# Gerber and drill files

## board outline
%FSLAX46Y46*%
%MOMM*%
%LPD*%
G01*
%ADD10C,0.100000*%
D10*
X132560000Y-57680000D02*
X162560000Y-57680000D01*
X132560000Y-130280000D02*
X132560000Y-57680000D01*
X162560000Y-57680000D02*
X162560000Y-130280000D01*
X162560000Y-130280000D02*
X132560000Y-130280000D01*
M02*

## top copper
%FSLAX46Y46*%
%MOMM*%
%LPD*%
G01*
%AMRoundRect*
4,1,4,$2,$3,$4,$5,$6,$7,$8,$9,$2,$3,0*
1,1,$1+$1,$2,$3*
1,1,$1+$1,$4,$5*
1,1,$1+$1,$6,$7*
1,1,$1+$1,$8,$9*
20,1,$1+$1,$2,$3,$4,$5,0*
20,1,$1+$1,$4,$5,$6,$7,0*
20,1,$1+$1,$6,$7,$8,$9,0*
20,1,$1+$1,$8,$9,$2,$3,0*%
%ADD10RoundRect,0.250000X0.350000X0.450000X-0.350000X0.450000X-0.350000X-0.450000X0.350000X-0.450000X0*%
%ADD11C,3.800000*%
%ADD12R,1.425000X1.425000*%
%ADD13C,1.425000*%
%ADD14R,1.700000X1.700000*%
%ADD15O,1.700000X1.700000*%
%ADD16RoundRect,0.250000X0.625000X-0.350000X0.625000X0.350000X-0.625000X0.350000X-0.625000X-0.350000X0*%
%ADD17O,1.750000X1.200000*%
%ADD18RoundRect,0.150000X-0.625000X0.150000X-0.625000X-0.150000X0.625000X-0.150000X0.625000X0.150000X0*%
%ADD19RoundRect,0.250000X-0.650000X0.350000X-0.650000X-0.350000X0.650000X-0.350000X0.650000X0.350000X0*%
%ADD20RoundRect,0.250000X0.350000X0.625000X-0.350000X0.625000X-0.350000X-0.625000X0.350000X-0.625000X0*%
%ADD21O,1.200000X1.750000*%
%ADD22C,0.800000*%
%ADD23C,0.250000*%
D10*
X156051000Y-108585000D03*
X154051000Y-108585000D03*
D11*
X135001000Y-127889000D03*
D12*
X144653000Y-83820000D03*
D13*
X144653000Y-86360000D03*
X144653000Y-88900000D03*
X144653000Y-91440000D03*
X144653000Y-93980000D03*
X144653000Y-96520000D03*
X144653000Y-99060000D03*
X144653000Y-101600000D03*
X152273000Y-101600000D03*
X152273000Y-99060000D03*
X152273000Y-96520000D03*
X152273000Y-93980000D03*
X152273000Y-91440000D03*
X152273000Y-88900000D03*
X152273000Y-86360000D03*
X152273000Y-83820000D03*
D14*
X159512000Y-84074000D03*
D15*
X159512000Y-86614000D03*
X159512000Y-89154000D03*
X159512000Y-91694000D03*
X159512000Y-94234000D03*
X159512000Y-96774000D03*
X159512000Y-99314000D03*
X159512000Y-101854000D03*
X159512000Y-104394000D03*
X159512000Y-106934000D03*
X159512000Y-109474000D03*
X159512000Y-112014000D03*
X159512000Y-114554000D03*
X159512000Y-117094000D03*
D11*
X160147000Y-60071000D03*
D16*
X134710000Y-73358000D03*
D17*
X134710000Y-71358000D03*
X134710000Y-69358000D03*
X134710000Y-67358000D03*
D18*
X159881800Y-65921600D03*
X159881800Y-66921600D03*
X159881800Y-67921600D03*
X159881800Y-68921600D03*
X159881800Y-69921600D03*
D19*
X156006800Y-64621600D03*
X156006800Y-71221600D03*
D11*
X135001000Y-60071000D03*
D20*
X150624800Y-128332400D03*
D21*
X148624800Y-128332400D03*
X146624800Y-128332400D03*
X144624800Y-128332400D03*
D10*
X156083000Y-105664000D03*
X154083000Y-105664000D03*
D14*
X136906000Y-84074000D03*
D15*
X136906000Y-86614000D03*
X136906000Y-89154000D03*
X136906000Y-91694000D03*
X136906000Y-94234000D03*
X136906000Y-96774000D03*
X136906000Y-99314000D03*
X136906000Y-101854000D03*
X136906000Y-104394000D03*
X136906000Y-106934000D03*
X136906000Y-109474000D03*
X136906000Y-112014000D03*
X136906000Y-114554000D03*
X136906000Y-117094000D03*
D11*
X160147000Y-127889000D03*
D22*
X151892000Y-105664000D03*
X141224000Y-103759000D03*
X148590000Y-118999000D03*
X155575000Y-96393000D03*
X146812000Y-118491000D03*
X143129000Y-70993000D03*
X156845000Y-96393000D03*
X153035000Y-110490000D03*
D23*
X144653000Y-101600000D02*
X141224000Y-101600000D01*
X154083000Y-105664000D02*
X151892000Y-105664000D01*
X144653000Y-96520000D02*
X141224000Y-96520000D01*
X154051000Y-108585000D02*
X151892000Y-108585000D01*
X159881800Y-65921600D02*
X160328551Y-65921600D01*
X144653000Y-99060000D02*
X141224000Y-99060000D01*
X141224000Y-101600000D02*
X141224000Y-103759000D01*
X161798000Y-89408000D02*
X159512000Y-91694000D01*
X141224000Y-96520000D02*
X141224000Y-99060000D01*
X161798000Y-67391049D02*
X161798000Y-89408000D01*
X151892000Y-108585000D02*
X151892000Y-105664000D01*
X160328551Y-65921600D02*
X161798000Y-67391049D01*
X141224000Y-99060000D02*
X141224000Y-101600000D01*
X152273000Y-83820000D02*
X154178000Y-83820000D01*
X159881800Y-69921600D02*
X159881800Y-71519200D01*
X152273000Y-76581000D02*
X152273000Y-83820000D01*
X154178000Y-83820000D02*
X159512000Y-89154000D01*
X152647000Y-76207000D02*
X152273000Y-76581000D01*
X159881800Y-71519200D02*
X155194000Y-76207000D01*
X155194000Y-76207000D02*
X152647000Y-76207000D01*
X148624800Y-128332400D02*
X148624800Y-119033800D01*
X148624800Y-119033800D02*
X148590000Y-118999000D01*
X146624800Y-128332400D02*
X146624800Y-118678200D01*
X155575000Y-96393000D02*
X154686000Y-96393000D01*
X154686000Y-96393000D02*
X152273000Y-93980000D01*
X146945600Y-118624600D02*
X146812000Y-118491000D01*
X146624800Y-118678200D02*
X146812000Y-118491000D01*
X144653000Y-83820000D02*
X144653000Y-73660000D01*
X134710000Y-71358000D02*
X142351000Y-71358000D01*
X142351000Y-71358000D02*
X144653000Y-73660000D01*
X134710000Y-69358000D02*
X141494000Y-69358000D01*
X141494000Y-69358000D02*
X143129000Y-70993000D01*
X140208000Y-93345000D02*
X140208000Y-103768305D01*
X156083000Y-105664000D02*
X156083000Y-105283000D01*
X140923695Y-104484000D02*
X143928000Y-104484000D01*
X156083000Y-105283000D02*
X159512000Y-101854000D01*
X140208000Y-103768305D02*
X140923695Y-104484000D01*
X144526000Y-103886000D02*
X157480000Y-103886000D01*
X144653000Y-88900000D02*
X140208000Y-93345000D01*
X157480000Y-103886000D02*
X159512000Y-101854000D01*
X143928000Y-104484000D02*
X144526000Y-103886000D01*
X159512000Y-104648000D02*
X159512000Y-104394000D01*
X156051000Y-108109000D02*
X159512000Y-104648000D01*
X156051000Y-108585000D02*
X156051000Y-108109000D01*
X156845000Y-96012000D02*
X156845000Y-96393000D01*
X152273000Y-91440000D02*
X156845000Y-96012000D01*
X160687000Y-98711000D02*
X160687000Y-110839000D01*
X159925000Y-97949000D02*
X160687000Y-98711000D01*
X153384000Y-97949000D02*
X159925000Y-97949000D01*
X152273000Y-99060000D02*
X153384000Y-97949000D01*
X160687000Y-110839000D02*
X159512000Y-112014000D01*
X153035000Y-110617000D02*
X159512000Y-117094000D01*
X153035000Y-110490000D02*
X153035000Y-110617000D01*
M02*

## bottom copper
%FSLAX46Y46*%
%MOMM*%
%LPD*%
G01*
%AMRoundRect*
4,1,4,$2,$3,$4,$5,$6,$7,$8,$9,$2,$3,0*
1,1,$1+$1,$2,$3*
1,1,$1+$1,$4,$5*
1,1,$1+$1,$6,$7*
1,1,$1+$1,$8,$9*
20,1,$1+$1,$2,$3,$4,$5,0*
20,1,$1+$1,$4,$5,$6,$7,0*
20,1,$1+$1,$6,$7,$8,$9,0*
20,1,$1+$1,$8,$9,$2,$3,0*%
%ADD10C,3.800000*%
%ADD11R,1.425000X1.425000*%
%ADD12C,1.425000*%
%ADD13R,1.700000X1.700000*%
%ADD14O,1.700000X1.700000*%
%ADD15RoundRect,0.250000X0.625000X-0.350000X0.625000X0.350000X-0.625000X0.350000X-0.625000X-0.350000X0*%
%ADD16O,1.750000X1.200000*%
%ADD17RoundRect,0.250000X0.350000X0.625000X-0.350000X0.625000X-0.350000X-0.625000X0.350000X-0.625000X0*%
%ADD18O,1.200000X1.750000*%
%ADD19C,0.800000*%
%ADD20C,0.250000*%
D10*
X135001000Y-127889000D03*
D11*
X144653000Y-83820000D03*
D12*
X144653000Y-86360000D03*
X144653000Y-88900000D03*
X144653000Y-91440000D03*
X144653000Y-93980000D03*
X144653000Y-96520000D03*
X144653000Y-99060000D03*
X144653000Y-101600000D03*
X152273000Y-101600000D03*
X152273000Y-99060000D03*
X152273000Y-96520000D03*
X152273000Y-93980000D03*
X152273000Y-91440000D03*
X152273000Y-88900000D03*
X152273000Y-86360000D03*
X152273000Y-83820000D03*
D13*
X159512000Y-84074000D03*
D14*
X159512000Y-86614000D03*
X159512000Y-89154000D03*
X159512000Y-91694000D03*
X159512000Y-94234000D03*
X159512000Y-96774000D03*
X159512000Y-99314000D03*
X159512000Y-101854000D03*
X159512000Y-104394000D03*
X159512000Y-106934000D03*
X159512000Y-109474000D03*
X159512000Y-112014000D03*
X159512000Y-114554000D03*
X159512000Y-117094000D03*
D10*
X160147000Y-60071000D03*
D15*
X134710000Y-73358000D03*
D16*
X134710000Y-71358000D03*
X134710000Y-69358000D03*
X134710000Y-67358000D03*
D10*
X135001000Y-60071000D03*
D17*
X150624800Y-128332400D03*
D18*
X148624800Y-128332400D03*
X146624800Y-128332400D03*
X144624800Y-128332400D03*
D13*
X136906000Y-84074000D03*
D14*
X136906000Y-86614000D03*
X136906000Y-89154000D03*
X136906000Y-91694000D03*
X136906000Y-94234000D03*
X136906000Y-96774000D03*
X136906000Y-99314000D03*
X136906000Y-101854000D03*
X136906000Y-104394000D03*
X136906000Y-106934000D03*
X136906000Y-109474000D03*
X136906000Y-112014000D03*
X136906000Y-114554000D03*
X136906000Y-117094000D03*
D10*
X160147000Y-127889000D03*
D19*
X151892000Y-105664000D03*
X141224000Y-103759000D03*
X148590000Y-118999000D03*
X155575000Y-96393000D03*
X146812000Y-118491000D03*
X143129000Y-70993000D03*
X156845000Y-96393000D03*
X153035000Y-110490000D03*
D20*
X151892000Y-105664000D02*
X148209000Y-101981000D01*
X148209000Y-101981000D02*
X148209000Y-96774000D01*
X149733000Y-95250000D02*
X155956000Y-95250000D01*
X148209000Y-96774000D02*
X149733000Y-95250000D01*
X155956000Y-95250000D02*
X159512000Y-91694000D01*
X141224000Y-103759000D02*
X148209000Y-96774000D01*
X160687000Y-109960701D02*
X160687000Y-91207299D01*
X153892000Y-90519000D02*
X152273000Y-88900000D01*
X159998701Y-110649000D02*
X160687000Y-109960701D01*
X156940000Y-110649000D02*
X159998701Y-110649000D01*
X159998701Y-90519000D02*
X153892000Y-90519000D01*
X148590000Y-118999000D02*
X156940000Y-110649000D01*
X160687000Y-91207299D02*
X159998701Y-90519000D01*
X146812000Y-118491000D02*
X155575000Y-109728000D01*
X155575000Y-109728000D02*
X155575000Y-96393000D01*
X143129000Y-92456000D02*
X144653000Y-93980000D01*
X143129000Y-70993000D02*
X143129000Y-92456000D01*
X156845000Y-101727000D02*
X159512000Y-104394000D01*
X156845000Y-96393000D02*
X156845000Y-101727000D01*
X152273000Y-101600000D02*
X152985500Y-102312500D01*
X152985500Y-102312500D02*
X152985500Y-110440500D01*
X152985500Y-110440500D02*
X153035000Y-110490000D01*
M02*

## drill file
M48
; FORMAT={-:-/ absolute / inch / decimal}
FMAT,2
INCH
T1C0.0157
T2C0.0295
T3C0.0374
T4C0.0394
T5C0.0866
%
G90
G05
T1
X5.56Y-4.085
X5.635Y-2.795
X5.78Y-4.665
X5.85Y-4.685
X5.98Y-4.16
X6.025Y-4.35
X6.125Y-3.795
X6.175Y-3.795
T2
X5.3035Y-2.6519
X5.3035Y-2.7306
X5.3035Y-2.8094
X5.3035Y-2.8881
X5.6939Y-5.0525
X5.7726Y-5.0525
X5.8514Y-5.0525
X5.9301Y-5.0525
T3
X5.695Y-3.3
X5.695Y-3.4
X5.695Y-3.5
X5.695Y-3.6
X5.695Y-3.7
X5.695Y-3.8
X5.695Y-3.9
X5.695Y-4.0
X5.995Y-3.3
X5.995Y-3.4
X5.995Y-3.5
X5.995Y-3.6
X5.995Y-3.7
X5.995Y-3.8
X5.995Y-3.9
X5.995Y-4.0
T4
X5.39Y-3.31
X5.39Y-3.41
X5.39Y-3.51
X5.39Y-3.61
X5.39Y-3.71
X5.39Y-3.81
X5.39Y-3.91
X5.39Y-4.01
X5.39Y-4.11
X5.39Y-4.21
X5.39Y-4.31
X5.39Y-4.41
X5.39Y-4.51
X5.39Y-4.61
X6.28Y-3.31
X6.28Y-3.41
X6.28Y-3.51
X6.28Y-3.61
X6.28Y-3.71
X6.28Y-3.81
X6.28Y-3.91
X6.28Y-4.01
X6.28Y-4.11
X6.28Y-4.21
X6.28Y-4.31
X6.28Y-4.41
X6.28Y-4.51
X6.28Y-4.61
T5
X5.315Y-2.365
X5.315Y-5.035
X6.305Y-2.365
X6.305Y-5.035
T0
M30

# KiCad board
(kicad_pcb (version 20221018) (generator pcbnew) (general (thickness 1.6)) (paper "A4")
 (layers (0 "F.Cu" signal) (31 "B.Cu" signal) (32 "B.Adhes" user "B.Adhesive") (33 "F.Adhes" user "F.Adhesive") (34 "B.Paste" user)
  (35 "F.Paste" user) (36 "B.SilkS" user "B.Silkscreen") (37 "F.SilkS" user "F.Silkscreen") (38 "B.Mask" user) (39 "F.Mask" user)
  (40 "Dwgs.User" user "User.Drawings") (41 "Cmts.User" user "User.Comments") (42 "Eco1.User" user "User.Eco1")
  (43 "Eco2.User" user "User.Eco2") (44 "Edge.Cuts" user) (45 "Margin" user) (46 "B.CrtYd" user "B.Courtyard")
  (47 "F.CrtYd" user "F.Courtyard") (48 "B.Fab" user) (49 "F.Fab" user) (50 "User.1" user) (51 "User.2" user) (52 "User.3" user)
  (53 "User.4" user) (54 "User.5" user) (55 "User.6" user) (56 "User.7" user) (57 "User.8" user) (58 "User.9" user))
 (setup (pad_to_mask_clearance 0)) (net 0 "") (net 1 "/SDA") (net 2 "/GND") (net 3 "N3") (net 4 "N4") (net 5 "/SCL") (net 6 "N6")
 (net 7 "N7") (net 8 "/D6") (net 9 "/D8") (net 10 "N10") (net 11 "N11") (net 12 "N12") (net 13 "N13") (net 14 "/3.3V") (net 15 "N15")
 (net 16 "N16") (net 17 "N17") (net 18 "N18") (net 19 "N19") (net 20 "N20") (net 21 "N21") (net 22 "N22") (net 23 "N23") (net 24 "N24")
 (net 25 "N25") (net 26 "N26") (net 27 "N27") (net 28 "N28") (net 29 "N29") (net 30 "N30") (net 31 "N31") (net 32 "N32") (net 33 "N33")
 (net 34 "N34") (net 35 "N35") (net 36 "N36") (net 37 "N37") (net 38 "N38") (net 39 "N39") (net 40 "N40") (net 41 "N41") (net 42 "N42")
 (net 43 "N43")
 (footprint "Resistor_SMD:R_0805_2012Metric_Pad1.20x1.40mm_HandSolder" (layer "F.Cu") (at 155.051 108.585 180)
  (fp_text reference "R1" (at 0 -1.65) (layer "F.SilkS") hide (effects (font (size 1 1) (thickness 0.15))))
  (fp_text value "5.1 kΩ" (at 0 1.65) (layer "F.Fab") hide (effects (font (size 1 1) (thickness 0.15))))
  (pad "1" smd roundrect (at -1 0 180) (size 1.2 1.4) (layers "F.Cu" "F.Paste" "F.Mask") (roundrect_rratio 0.2083333333) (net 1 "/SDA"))
  (pad "2" smd roundrect (at 1 0 180) (size 1.2 1.4) (layers "F.Cu" "F.Paste" "F.Mask") (roundrect_rratio 0.2083333333) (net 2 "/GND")))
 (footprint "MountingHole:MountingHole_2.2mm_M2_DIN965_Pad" (layer "F.Cu") (at 135.001 127.889)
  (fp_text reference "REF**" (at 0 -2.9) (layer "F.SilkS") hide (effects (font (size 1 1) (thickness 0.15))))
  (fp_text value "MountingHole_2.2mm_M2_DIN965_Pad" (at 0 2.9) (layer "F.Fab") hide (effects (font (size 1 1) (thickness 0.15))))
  (pad "1" thru_hole circle (at 0 0) (size 3.8 3.8) (drill 2.2) (layers "*.Cu" "*.Mask")))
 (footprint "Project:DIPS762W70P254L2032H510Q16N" (layer "F.Cu") (at 144.653 83.82)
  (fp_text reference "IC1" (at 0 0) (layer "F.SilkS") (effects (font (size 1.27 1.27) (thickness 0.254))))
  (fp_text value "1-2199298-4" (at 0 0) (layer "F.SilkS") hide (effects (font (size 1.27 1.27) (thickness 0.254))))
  (pad "1" thru_hole rect (at 0 0) (size 1.425 1.425) (drill 0.95) (layers "*.Cu" "*.Mask") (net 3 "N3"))
  (pad "2" thru_hole circle (at 0 2.54) (size 1.425 1.425) (drill 0.95) (layers "*.Cu" "*.Mask") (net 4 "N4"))
  (pad "3" thru_hole circle (at 0 5.08) (size 1.425 1.425) (drill 0.95) (layers "*.Cu" "*.Mask") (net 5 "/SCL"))
  (pad "4" thru_hole circle (at 0 7.62) (size 1.425 1.425) (drill 0.95) (layers "*.Cu" "*.Mask") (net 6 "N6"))
  (pad "5" thru_hole circle (at 0 10.16) (size 1.425 1.425) (drill 0.95) (layers "*.Cu" "*.Mask") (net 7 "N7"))
  (pad "6" thru_hole circle (at 0 12.7) (size 1.425 1.425) (drill 0.95) (layers "*.Cu" "*.Mask") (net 2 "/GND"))
  (pad "7" thru_hole circle (at 0 15.24) (size 1.425 1.425) (drill 0.95) (layers "*.Cu" "*.Mask") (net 2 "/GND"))
  (pad "8" thru_hole circle (at 0 17.78) (size 1.425 1.425) (drill 0.95) (layers "*.Cu" "*.Mask") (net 2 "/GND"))
  (pad "9" thru_hole circle (at 7.62 17.78) (size 1.425 1.425) (drill 0.95) (layers "*.Cu" "*.Mask") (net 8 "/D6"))
  (pad "10" thru_hole circle (at 7.62 15.24) (size 1.425 1.425) (drill 0.95) (layers "*.Cu" "*.Mask") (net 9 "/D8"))
  (pad "11" thru_hole circle (at 7.62 12.7) (size 1.425 1.425) (drill 0.95) (layers "*.Cu" "*.Mask") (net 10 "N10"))
  (pad "12" thru_hole circle (at 7.62 10.16) (size 1.425 1.425) (drill 0.95) (layers "*.Cu" "*.Mask") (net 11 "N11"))
  (pad "13" thru_hole circle (at 7.62 7.62) (size 1.425 1.425) (drill 0.95) (layers "*.Cu" "*.Mask") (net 1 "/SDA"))
  (pad "14" thru_hole circle (at 7.62 5.08) (size 1.425 1.425) (drill 0.95) (layers "*.Cu" "*.Mask") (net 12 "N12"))
  (pad "15" thru_hole circle (at 7.62 2.54) (size 1.425 1.425) (drill 0.95) (layers "*.Cu" "*.Mask") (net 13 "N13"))
  (pad "16" thru_hole circle (at 7.62 0) (size 1.425 1.425) (drill 0.95) (layers "*.Cu" "*.Mask") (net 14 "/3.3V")))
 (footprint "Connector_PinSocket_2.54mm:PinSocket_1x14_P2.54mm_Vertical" (layer "F.Cu") (at 159.512 84.074)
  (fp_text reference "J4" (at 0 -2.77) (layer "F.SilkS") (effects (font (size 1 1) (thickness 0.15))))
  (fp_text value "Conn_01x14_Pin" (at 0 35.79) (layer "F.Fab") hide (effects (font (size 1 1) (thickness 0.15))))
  (pad "1" thru_hole rect (at 0 0) (size 1.7 1.7) (drill 1) (layers "*.Cu" "*.Mask") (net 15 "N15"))
  (pad "2" thru_hole oval (at 0 2.54) (size 1.7 1.7) (drill 1) (layers "*.Cu" "*.Mask") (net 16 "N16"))
  (pad "3" thru_hole oval (at 0 5.08) (size 1.7 1.7) (drill 1) (layers "*.Cu" "*.Mask") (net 14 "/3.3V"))
  (pad "4" thru_hole oval (at 0 7.62) (size 1.7 1.7) (drill 1) (layers "*.Cu" "*.Mask") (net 2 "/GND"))
  (pad "5" thru_hole oval (at 0 10.16) (size 1.7 1.7) (drill 1) (layers "*.Cu" "*.Mask") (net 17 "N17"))
  (pad "6" thru_hole oval (at 0 12.7) (size 1.7 1.7) (drill 1) (layers "*.Cu" "*.Mask") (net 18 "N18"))
  (pad "7" thru_hole oval (at 0 15.24) (size 1.7 1.7) (drill 1) (layers "*.Cu" "*.Mask") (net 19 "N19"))
  (pad "8" thru_hole oval (at 0 17.78) (size 1.7 1.7) (drill 1) (layers "*.Cu" "*.Mask") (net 5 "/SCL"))
  (pad "9" thru_hole oval (at 0 20.32) (size 1.7 1.7) (drill 1) (layers "*.Cu" "*.Mask") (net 1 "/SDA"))
  (pad "10" thru_hole oval (at 0 22.86) (size 1.7 1.7) (drill 1) (layers "*.Cu" "*.Mask") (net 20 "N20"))
  (pad "11" thru_hole oval (at 0 25.4) (size 1.7 1.7) (drill 1) (layers "*.Cu" "*.Mask") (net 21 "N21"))
  (pad "12" thru_hole oval (at 0 27.94) (size 1.7 1.7) (drill 1) (layers "*.Cu" "*.Mask") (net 9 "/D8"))
  (pad "13" thru_hole oval (at 0 30.48) (size 1.7 1.7) (drill 1) (layers "*.Cu" "*.Mask") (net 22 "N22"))
  (pad "14" thru_hole oval (at 0 33.02) (size 1.7 1.7) (drill 1) (layers "*.Cu" "*.Mask") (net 8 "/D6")))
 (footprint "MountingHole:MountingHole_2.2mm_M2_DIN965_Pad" (layer "F.Cu") (at 160.147 60.071)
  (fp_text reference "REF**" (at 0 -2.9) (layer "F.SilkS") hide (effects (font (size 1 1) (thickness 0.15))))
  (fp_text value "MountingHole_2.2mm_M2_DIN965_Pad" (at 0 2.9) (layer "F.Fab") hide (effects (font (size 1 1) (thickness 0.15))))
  (pad "1" thru_hole circle (at 0 0) (size 3.8 3.8) (drill 2.2) (layers "*.Cu" "*.Mask")))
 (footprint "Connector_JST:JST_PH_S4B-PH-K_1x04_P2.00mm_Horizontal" (layer "F.Cu") (at 134.71 73.358 90)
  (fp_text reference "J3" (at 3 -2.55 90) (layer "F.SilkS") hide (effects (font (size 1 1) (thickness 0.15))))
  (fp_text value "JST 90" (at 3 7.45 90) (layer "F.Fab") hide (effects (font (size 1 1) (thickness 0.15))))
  (pad "1" thru_hole roundrect (at 0 0 90) (size 1.2 1.75) (drill 0.75) (layers "*.Cu" "*.Mask") (roundrect_rratio 0.2083333333)
   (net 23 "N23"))
  (pad "2" thru_hole oval (at 2 0 90) (size 1.2 1.75) (drill 0.75) (layers "*.Cu" "*.Mask") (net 3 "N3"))
  (pad "3" thru_hole oval (at 4 0 90) (size 1.2 1.75) (drill 0.75) (layers "*.Cu" "*.Mask") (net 7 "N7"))
  (pad "4" thru_hole oval (at 6 0 90) (size 1.2 1.75) (drill 0.75) (layers "*.Cu" "*.Mask") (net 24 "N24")))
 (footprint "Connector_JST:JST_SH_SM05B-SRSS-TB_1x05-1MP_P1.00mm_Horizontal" (layer "F.Cu") (at 157.8818 67.9216 -90)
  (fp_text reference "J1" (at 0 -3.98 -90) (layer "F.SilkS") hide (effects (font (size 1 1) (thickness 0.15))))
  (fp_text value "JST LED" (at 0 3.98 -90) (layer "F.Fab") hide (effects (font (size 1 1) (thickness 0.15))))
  (pad "1" smd roundrect (at -2 -2 270) (size 0.6 1.55) (layers "F.Cu" "F.Paste" "F.Mask") (roundrect_rratio 0.25) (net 2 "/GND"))
  (pad "2" smd roundrect (at -1 -2 270) (size 0.6 1.55) (layers "F.Cu" "F.Paste" "F.Mask") (roundrect_rratio 0.25) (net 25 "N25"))
  (pad "3" smd roundrect (at 0 -2 270) (size 0.6 1.55) (layers "F.Cu" "F.Paste" "F.Mask") (roundrect_rratio 0.25) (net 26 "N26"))
  (pad "4" smd roundrect (at 1 -2 270) (size 0.6 1.55) (layers "F.Cu" "F.Paste" "F.Mask") (roundrect_rratio 0.25) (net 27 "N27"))
  (pad "5" smd roundrect (at 2 -2 270) (size 0.6 1.55) (layers "F.Cu" "F.Paste" "F.Mask") (roundrect_rratio 0.25) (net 14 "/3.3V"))
  (pad "MP" smd roundrect (at -3.3 1.875 270) (size 1.2 1.8) (layers "F.Cu" "F.Paste" "F.Mask") (roundrect_rratio 0.2083333333))
  (pad "MP" smd roundrect (at 3.3 1.875 270) (size 1.2 1.8) (layers "F.Cu" "F.Paste" "F.Mask") (roundrect_rratio 0.2083333333)))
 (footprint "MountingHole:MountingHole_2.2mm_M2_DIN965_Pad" (layer "F.Cu") (at 135.001 60.071)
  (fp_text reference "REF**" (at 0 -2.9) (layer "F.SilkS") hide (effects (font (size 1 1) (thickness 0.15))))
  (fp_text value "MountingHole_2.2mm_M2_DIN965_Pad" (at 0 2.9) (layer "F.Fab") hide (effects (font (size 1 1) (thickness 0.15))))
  (pad "1" thru_hole circle (at 0 0) (size 3.8 3.8) (drill 2.2) (layers "*.Cu" "*.Mask")))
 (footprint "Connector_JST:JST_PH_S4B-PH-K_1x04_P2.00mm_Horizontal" (layer "F.Cu") (at 150.6248 128.3324 180)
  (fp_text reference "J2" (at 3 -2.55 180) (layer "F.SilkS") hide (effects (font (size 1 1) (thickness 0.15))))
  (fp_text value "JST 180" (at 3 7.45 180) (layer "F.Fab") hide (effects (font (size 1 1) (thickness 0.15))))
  (pad "1" thru_hole roundrect (at 0 0 180) (size 1.2 1.75) (drill 0.75) (layers "*.Cu" "*.Mask") (roundrect_rratio 0.2083333333)
   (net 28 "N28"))
  (pad "2" thru_hole oval (at 2 0 180) (size 1.2 1.75) (drill 0.75) (layers "*.Cu" "*.Mask") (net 12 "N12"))
  (pad "3" thru_hole oval (at 4 0 180) (size 1.2 1.75) (drill 0.75) (layers "*.Cu" "*.Mask") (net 11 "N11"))
  (pad "4" thru_hole oval (at 6 0 180) (size 1.2 1.75) (drill 0.75) (layers "*.Cu" "*.Mask") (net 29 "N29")))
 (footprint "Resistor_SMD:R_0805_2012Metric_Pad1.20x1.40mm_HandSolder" (layer "F.Cu") (at 155.083 105.664 180)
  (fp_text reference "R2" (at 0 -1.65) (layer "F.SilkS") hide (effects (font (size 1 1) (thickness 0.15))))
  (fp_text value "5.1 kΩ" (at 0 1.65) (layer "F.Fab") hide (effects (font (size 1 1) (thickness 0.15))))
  (pad "1" smd roundrect (at -1 0 180) (size 1.2 1.4) (layers "F.Cu" "F.Paste" "F.Mask") (roundrect_rratio 0.2083333333) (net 5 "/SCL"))
  (pad "2" smd roundrect (at 1 0 180) (size 1.2 1.4) (layers "F.Cu" "F.Paste" "F.Mask") (roundrect_rratio 0.2083333333) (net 2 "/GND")))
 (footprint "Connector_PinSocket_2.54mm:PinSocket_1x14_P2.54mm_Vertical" (layer "F.Cu") (at 136.906 84.074)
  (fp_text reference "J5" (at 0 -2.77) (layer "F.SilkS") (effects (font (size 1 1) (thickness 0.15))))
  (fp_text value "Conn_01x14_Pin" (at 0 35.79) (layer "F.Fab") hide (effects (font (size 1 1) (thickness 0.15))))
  (pad "1" thru_hole rect (at 0 0) (size 1.7 1.7) (drill 1) (layers "*.Cu" "*.Mask") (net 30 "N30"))
  (pad "2" thru_hole oval (at 0 2.54) (size 1.7 1.7) (drill 1) (layers "*.Cu" "*.Mask") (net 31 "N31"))
  (pad "3" thru_hole oval (at 0 5.08) (size 1.7 1.7) (drill 1) (layers "*.Cu" "*.Mask") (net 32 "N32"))
  (pad "4" thru_hole oval (at 0 7.62) (size 1.7 1.7) (drill 1) (layers "*.Cu" "*.Mask") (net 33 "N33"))
  (pad "5" thru_hole oval (at 0 10.16) (size 1.7 1.7) (drill 1) (layers "*.Cu" "*.Mask") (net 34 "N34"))
  (pad "6" thru_hole oval (at 0 12.7) (size 1.7 1.7) (drill 1) (layers "*.Cu" "*.Mask") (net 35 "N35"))
  (pad "7" thru_hole oval (at 0 15.24) (size 1.7 1.7) (drill 1) (layers "*.Cu" "*.Mask") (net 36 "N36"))
  (pad "8" thru_hole oval (at 0 17.78) (size 1.7 1.7) (drill 1) (layers "*.Cu" "*.Mask") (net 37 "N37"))
  (pad "9" thru_hole oval (at 0 20.32) (size 1.7 1.7) (drill 1) (layers "*.Cu" "*.Mask") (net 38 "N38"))
  (pad "10" thru_hole oval (at 0 22.86) (size 1.7 1.7) (drill 1) (layers "*.Cu" "*.Mask") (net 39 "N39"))
  (pad "11" thru_hole oval (at 0 25.4) (size 1.7 1.7) (drill 1) (layers "*.Cu" "*.Mask") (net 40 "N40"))
  (pad "12" thru_hole oval (at 0 27.94) (size 1.7 1.7) (drill 1) (layers "*.Cu" "*.Mask") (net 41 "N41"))
  (pad "13" thru_hole oval (at 0 30.48) (size 1.7 1.7) (drill 1) (layers "*.Cu" "*.Mask") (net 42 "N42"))
  (pad "14" thru_hole oval (at 0 33.02) (size 1.7 1.7) (drill 1) (layers "*.Cu" "*.Mask") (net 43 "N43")))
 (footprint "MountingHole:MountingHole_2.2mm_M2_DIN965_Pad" (layer "F.Cu") (at 160.147 127.889)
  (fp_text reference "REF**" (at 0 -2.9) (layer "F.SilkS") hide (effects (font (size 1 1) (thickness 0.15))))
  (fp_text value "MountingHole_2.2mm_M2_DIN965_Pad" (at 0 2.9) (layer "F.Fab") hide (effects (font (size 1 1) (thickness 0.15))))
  (pad "1" thru_hole circle (at 0 0) (size 3.8 3.8) (drill 2.2) (layers "*.Cu" "*.Mask")))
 (gr_line (start 132.56 57.68) (end 162.56 57.68) (stroke (width 0.1) (type default)) (layer "Edge.Cuts"))
 (gr_line (start 132.56 130.28) (end 132.56 57.68) (stroke (width 0.1) (type default)) (layer "Edge.Cuts"))
 (gr_line (start 162.56 57.68) (end 162.56 130.28) (stroke (width 0.1) (type default)) (layer "Edge.Cuts"))
 (gr_line (start 162.56 130.28) (end 132.56 130.28) (stroke (width 0.1) (type default)) (layer "Edge.Cuts"))
 (segment (start 144.653 101.6) (end 141.224 101.6) (width 0.25) (layer "F.Cu") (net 2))
 (segment (start 154.083 105.664) (end 151.892 105.664) (width 0.25) (layer "F.Cu") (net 2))
 (segment (start 144.653 96.52) (end 141.224 96.52) (width 0.25) (layer "F.Cu") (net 2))
 (segment (start 154.051 108.585) (end 151.892 108.585) (width 0.25) (layer "F.Cu") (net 2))
 (segment (start 159.8818 65.9216) (end 160.328551 65.9216) (width 0.25) (layer "F.Cu") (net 2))
 (segment (start 144.653 99.06) (end 141.224 99.06) (width 0.25) (layer "F.Cu") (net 2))
 (segment (start 141.224 101.6) (end 141.224 103.759) (width 0.25) (layer "F.Cu") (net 2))
 (segment (start 161.798 89.408) (end 159.512 91.694) (width 0.25) (layer "F.Cu") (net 2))
 (segment (start 141.224 96.52) (end 141.224 99.06) (width 0.25) (layer "F.Cu") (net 2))
 (segment (start 161.798 67.391049) (end 161.798 89.408) (width 0.25) (layer "F.Cu") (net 2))
 (segment (start 151.892 108.585) (end 151.892 105.664) (width 0.25) (layer "F.Cu") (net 2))
 (segment (start 160.328551 65.9216) (end 161.798 67.391049) (width 0.25) (layer "F.Cu") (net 2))
 (segment (start 141.224 99.06) (end 141.224 101.6) (width 0.25) (layer "F.Cu") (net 2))
 (via (at 151.892 105.664) (size 0.8) (drill 0.4) (layers "F.Cu" "B.Cu") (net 2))
 (via (at 141.224 103.759) (size 0.8) (drill 0.4) (layers "F.Cu" "B.Cu") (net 2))
 (segment (start 151.892 105.664) (end 148.209 101.981) (width 0.25) (layer "B.Cu") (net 2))
 (segment (start 148.209 101.981) (end 148.209 96.774) (width 0.25) (layer "B.Cu") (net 2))
 (segment (start 149.733 95.25) (end 155.956 95.25) (width 0.25) (layer "B.Cu") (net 2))
 (segment (start 148.209 96.774) (end 149.733 95.25) (width 0.25) (layer "B.Cu") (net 2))
 (segment (start 155.956 95.25) (end 159.512 91.694) (width 0.25) (layer "B.Cu") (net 2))
 (segment (start 141.224 103.759) (end 148.209 96.774) (width 0.25) (layer "B.Cu") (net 2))
 (segment (start 152.273 83.82) (end 154.178 83.82) (width 0.25) (layer "F.Cu") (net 14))
 (segment (start 159.8818 69.9216) (end 159.8818 71.5192) (width 0.25) (layer "F.Cu") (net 14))
 (segment (start 152.273 76.581) (end 152.273 83.82) (width 0.25) (layer "F.Cu") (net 14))
 (segment (start 154.178 83.82) (end 159.512 89.154) (width 0.25) (layer "F.Cu") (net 14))
 (segment (start 152.647 76.207) (end 152.273 76.581) (width 0.25) (layer "F.Cu") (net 14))
 (segment (start 159.8818 71.5192) (end 155.194 76.207) (width 0.25) (layer "F.Cu") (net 14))
 (segment (start 155.194 76.207) (end 152.647 76.207) (width 0.25) (layer "F.Cu") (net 14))
 (segment (start 148.6248 128.3324) (end 148.6248 119.0338) (width 0.25) (layer "F.Cu") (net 12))
 (segment (start 148.6248 119.0338) (end 148.59 118.999) (width 0.25) (layer "F.Cu") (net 12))
 (via (at 148.59 118.999) (size 0.8) (drill 0.4) (layers "F.Cu" "B.Cu") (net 12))
 (segment (start 160.687 109.960701) (end 160.687 91.207299) (width 0.25) (layer "B.Cu") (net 12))
 (segment (start 153.892 90.519) (end 152.273 88.9) (width 0.25) (layer "B.Cu") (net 12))
 (segment (start 159.998701 110.649) (end 160.687 109.960701) (width 0.25) (layer "B.Cu") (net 12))
 (segment (start 156.94 110.649) (end 159.998701 110.649) (width 0.25) (layer "B.Cu") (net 12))
 (segment (start 159.998701 90.519) (end 153.892 90.519) (width 0.25) (layer "B.Cu") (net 12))
 (segment (start 148.59 118.999) (end 156.94 110.649) (width 0.25) (layer "B.Cu") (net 12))
 (segment (start 160.687 91.207299) (end 159.998701 90.519) (width 0.25) (layer "B.Cu") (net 12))
 (segment (start 146.6248 128.3324) (end 146.6248 118.6782) (width 0.25) (layer "F.Cu") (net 11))
 (segment (start 155.575 96.393) (end 154.686 96.393) (width 0.25) (layer "F.Cu") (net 11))
 (segment (start 154.686 96.393) (end 152.273 93.98) (width 0.25) (layer "F.Cu") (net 11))
 (segment (start 146.9456 118.6246) (end 146.812 118.491) (width 0.25) (layer "F.Cu") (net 11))
 (segment (start 146.6248 118.6782) (end 146.812 118.491) (width 0.25) (layer "F.Cu") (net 11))
 (via (at 155.575 96.393) (size 0.8) (drill 0.4) (layers "F.Cu" "B.Cu") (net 11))
 (via (at 146.812 118.491) (size 0.8) (drill 0.4) (layers "F.Cu" "B.Cu") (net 11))
 (segment (start 146.812 118.491) (end 155.575 109.728) (width 0.25) (layer "B.Cu") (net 11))
 (segment (start 155.575 109.728) (end 155.575 96.393) (width 0.25) (layer "B.Cu") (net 11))
 (segment (start 144.653 83.82) (end 144.653 73.66) (width 0.25) (layer "F.Cu") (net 3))
 (segment (start 134.71 71.358) (end 142.351 71.358) (width 0.25) (layer "F.Cu") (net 3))
 (segment (start 142.351 71.358) (end 144.653 73.66) (width 0.25) (layer "F.Cu") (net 3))
 (segment (start 134.71 69.358) (end 141.494 69.358) (width 0.25) (layer "F.Cu") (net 7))
 (segment (start 141.494 69.358) (end 143.129 70.993) (width 0.25) (layer "F.Cu") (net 7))
 (via (at 143.129 70.993) (size 0.8) (drill 0.4) (layers "F.Cu" "B.Cu") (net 7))
 (segment (start 143.129 92.456) (end 144.653 93.98) (width 0.25) (layer "B.Cu") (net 7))
 (segment (start 143.129 70.993) (end 143.129 92.456) (width 0.25) (layer "B.Cu") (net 7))
 (segment (start 140.208 93.345) (end 140.208 103.768305) (width 0.25) (layer "F.Cu") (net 5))
 (segment (start 156.083 105.664) (end 156.083 105.283) (width 0.25) (layer "F.Cu") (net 5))
 (segment (start 140.923695 104.484) (end 143.928 104.484) (width 0.25) (layer "F.Cu") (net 5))
 (segment (start 156.083 105.283) (end 159.512 101.854) (width 0.25) (layer "F.Cu") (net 5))
 (segment (start 140.208 103.768305) (end 140.923695 104.484) (width 0.25) (layer "F.Cu") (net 5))
 (segment (start 144.526 103.886) (end 157.48 103.886) (width 0.25) (layer "F.Cu") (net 5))
 (segment (start 144.653 88.9) (end 140.208 93.345) (width 0.25) (layer "F.Cu") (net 5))
 (segment (start 157.48 103.886) (end 159.512 101.854) (width 0.25) (layer "F.Cu") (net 5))
 (segment (start 143.928 104.484) (end 144.526 103.886) (width 0.25) (layer "F.Cu") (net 5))
 (segment (start 159.512 104.648) (end 159.512 104.394) (width 0.25) (layer "F.Cu") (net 1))
 (segment (start 156.051 108.109) (end 159.512 104.648) (width 0.25) (layer "F.Cu") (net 1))
 (segment (start 156.051 108.585) (end 156.051 108.109) (width 0.25) (layer "F.Cu") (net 1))
 (segment (start 156.845 96.012) (end 156.845 96.393) (width 0.25) (layer "F.Cu") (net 1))
 (segment (start 152.273 91.44) (end 156.845 96.012) (width 0.25) (layer "F.Cu") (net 1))
 (via (at 156.845 96.393) (size 0.8) (drill 0.4) (layers "F.Cu" "B.Cu") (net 1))
 (segment (start 156.845 101.727) (end 159.512 104.394) (width 0.25) (layer "B.Cu") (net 1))
 (segment (start 156.845 96.393) (end 156.845 101.727) (width 0.25) (layer "B.Cu") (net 1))
 (segment (start 160.687 98.711) (end 160.687 110.839) (width 0.25) (layer "F.Cu") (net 9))
 (segment (start 159.925 97.949) (end 160.687 98.711) (width 0.25) (layer "F.Cu") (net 9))
 (segment (start 153.384 97.949) (end 159.925 97.949) (width 0.25) (layer "F.Cu") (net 9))
 (segment (start 152.273 99.06) (end 153.384 97.949) (width 0.25) (layer "F.Cu") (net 9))
 (segment (start 160.687 110.839) (end 159.512 112.014) (width 0.25) (layer "F.Cu") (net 9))
 (segment (start 153.035 110.617) (end 159.512 117.094) (width 0.25) (layer "F.Cu") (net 8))
 (segment (start 153.035 110.49) (end 153.035 110.617) (width 0.25) (layer "F.Cu") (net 8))
 (via (at 153.035 110.49) (size 0.8) (drill 0.4) (layers "F.Cu" "B.Cu") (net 8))
 (segment (start 152.273 101.6) (end 152.9855 102.3125) (width 0.25) (layer "B.Cu") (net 8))
 (segment (start 152.9855 102.3125) (end 152.9855 110.4405) (width 0.25) (layer "B.Cu") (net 8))
 (segment (start 152.9855 110.4405) (end 153.035 110.49) (width 0.25) (layer "B.Cu") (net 8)))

